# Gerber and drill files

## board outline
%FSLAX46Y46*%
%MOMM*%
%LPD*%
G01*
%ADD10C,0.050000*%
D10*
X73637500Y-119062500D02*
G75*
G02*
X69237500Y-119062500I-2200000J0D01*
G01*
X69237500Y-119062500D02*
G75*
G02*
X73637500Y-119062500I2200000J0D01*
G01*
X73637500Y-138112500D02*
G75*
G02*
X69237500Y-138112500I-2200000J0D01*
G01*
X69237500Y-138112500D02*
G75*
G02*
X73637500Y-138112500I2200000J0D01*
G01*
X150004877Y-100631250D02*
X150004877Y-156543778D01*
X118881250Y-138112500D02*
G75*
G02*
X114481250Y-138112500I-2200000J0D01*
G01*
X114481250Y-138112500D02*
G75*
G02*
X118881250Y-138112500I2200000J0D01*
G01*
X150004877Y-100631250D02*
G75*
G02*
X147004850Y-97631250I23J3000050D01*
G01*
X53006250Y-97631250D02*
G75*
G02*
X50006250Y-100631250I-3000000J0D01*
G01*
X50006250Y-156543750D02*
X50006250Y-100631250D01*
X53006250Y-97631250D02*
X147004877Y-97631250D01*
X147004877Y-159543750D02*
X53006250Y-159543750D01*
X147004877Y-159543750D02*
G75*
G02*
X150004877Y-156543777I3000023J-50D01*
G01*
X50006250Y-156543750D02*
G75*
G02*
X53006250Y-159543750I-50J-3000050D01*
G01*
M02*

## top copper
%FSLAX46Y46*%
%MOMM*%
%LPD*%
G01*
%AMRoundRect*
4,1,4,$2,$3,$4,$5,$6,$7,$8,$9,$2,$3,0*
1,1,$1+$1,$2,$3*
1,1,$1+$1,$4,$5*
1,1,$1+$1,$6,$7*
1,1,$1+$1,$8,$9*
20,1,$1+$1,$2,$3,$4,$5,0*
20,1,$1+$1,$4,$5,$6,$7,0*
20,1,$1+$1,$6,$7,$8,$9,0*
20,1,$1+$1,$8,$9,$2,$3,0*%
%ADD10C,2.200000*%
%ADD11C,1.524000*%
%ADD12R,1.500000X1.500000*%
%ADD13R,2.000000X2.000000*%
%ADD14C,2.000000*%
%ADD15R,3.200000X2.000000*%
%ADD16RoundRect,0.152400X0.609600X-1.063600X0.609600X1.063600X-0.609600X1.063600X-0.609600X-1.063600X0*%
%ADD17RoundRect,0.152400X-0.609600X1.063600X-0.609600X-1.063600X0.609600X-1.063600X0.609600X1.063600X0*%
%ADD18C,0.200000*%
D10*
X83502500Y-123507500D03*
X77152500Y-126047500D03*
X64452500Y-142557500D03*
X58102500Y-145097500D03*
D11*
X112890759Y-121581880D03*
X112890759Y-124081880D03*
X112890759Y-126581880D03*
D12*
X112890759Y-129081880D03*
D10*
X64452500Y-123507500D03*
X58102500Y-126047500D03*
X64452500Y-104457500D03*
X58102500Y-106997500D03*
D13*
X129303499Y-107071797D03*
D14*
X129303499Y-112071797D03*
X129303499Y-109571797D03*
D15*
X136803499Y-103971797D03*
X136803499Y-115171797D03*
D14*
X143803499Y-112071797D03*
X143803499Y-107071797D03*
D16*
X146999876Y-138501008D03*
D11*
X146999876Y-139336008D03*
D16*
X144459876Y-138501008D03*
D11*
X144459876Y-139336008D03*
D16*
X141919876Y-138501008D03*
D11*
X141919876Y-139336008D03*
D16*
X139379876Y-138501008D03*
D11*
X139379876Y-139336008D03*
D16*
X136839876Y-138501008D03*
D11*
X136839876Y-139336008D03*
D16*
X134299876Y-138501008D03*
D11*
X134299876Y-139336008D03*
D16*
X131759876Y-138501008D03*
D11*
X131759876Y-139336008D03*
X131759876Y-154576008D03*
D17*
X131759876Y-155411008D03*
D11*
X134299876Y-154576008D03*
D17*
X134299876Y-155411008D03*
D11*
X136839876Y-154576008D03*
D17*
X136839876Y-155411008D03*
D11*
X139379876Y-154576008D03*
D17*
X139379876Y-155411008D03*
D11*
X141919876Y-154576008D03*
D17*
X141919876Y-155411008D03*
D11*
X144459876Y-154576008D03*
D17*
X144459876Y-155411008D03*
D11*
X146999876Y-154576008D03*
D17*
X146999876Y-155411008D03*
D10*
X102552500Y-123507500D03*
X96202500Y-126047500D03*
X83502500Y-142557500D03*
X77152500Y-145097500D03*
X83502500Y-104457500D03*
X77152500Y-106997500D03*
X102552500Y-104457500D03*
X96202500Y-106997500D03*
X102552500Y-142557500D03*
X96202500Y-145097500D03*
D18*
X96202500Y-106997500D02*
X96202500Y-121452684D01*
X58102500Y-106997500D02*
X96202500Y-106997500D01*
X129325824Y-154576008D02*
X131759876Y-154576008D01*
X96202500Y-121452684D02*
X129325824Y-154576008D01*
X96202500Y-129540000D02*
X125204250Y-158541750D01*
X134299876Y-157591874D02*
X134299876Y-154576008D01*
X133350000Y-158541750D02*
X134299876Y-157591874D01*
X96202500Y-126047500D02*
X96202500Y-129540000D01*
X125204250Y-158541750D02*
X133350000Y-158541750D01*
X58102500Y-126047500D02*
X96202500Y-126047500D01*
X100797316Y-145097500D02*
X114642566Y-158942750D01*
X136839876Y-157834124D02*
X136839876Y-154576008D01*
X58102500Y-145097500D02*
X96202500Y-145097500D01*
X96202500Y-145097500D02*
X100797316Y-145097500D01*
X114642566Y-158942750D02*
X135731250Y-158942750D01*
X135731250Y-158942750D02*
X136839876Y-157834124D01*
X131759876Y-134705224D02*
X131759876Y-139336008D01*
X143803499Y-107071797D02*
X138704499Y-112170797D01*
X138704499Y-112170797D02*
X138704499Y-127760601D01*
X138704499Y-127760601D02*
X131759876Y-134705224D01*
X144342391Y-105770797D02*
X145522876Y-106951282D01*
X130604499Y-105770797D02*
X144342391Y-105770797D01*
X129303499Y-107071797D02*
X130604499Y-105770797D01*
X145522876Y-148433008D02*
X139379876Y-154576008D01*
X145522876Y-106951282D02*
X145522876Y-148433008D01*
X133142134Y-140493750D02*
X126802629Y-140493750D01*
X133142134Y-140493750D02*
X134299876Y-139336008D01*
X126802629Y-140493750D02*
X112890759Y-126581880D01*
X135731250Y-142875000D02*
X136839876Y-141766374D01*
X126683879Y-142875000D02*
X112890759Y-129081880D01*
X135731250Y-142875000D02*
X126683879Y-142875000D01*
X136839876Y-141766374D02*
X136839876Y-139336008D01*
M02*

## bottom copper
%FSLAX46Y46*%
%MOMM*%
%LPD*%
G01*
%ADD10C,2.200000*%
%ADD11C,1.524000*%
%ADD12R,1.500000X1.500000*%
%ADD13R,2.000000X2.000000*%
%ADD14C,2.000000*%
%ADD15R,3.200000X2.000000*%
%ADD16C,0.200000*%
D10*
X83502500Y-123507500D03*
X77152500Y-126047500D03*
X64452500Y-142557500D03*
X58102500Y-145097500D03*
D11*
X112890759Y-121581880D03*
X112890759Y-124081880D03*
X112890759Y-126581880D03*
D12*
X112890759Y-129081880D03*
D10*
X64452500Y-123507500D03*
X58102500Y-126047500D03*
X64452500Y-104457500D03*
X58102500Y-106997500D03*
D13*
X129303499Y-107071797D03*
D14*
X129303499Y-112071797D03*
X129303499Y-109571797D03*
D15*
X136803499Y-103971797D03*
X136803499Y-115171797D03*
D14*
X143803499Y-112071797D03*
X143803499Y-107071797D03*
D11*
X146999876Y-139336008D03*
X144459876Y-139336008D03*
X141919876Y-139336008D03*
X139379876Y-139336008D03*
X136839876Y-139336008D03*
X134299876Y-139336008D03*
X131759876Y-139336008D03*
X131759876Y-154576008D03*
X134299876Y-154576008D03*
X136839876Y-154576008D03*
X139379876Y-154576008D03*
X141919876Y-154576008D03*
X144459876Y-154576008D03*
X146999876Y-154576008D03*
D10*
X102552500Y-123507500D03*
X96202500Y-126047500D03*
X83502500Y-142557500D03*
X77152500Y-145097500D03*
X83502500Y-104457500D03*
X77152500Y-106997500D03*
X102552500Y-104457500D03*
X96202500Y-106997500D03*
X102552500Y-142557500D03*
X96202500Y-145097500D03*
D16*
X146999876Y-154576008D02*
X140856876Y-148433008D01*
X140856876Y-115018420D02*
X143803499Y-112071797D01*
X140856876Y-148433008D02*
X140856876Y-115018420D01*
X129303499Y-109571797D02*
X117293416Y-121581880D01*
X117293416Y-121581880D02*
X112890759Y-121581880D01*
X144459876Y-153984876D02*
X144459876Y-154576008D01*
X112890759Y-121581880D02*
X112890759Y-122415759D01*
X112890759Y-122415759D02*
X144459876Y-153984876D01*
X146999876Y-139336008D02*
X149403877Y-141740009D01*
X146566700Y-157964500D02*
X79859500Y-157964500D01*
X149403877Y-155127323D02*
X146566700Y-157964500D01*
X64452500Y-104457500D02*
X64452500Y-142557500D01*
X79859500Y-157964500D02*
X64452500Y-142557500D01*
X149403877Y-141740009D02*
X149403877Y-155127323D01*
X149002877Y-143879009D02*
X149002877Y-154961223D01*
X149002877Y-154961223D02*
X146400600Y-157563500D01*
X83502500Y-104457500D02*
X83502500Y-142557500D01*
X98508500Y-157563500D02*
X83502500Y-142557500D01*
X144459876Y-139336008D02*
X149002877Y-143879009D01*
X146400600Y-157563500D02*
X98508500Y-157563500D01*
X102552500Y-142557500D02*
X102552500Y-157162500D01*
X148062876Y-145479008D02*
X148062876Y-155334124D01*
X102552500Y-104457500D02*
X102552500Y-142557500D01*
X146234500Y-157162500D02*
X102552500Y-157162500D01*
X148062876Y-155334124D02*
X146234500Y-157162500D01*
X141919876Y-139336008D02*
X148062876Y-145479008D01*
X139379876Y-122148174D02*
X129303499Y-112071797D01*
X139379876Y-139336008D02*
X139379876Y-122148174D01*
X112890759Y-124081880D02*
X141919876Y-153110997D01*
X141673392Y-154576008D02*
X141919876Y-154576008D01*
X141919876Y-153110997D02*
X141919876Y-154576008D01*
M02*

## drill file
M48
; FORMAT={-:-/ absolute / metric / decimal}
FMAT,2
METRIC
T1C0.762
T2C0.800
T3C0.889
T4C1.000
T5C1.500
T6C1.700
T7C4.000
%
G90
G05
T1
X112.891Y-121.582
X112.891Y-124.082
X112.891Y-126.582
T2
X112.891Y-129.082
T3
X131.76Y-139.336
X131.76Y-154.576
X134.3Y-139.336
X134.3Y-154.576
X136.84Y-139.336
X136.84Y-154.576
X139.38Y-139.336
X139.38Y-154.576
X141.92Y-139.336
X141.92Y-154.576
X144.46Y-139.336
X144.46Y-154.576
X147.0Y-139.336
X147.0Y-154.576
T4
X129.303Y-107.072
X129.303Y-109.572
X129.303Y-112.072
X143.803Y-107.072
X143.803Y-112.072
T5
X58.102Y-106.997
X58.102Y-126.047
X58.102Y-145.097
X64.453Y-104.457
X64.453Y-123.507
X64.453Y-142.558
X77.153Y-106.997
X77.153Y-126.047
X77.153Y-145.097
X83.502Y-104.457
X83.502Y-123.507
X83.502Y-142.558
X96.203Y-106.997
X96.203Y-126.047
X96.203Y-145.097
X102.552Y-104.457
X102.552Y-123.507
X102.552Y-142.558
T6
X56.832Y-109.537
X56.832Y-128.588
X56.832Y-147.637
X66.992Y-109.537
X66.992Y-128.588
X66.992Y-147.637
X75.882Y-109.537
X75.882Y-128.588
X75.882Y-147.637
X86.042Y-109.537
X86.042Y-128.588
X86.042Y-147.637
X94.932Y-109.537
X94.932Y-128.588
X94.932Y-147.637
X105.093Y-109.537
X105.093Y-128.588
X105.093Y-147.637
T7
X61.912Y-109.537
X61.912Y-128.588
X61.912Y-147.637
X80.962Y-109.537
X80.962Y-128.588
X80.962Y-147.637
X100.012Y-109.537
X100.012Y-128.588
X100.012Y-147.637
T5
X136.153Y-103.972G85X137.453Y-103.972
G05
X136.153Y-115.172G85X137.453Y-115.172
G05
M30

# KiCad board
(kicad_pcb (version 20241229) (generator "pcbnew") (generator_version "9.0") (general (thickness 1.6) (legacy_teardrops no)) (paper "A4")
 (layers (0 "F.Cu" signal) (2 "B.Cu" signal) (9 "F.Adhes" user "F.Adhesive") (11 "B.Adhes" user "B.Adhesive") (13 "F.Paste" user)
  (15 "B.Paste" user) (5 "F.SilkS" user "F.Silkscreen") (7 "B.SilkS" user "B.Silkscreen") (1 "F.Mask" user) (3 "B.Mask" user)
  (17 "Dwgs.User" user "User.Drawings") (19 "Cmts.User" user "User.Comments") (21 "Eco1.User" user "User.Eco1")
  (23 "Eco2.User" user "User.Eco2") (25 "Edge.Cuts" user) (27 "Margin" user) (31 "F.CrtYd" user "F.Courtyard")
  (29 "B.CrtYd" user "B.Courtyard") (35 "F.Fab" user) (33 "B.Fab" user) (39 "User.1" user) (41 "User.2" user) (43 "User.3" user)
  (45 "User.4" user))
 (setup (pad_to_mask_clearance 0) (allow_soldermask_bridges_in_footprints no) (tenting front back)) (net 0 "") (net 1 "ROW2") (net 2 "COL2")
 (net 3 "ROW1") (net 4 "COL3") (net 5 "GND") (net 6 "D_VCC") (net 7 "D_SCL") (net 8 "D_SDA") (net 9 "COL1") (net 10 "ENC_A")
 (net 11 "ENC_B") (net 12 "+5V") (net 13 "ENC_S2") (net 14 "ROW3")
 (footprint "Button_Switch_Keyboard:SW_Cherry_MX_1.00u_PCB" (layer "F.Cu") (at 83.5025 123.5075)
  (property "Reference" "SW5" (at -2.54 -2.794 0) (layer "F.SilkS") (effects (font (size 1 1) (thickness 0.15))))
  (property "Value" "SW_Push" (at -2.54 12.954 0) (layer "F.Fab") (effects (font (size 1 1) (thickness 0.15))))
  (pad "" np_thru_hole circle (at -7.62 5.08) (size 1.7 1.7) (drill 1.7) (layers "*.Cu" "*.Mask"))
  (pad "" np_thru_hole circle (at -2.54 5.08) (size 4 4) (drill 4) (layers "*.Cu" "*.Mask"))
  (pad "" np_thru_hole circle (at 2.54 5.08) (size 1.7 1.7) (drill 1.7) (layers "*.Cu" "*.Mask"))
  (pad "1" thru_hole circle (at 0 0) (size 2.2 2.2) (drill 1.5) (layers "*.Cu" "*.Mask") (remove_unused_layers no) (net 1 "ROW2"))
  (pad "2" thru_hole circle (at -6.35 2.54) (size 2.2 2.2) (drill 1.5) (layers "*.Cu" "*.Mask") (remove_unused_layers no) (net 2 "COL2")))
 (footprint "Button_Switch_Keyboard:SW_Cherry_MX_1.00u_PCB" (layer "F.Cu") (at 64.4525 142.5575)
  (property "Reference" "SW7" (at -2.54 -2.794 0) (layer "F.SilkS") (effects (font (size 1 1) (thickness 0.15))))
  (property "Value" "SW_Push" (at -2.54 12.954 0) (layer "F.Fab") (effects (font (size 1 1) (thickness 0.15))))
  (pad "" np_thru_hole circle (at -7.62 5.08) (size 1.7 1.7) (drill 1.7) (layers "*.Cu" "*.Mask"))
  (pad "" np_thru_hole circle (at -2.54 5.08) (size 4 4) (drill 4) (layers "*.Cu" "*.Mask"))
  (pad "" np_thru_hole circle (at 2.54 5.08) (size 1.7 1.7) (drill 1.7) (layers "*.Cu" "*.Mask"))
  (pad "1" thru_hole circle (at 0 0) (size 2.2 2.2) (drill 1.5) (layers "*.Cu" "*.Mask") (remove_unused_layers no) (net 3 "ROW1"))
  (pad "2" thru_hole circle (at -6.35 2.54) (size 2.2 2.2) (drill 1.5) (layers "*.Cu" "*.Mask") (remove_unused_layers no) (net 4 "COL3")))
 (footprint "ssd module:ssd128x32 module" (layer "F.Cu") (at 126.12851 139.246137)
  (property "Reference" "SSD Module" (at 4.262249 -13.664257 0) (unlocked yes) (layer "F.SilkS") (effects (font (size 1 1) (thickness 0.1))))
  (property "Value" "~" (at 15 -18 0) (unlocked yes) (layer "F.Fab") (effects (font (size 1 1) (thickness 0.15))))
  (pad "1" thru_hole circle (at -13.237751 -17.664257) (size 1.524 1.524) (drill 0.762) (layers "*.Cu" "*.Mask") (remove_unused_layers no)
   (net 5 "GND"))
  (pad "2" thru_hole circle (at -13.237751 -15.164257) (size 1.524 1.524) (drill 0.762) (layers "*.Cu" "*.Mask") (remove_unused_layers no)
   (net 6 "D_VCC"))
  (pad "3" thru_hole circle (at -13.237751 -12.664257) (size 1.524 1.524) (drill 0.762) (layers "*.Cu" "*.Mask") (remove_unused_layers no)
   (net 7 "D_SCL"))
  (pad "4" thru_hole rect (at -13.237751 -10.164257) (size 1.5 1.5) (drill 0.8) (layers "*.Cu" "*.Mask") (remove_unused_layers no)
   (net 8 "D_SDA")))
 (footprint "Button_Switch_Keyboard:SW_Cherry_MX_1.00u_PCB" (layer "F.Cu") (at 64.4525 123.5075)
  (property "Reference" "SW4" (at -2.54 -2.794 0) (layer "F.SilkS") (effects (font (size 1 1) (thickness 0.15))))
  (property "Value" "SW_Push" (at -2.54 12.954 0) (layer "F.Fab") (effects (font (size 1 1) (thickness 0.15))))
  (pad "" np_thru_hole circle (at -7.62 5.08) (size 1.7 1.7) (drill 1.7) (layers "*.Cu" "*.Mask"))
  (pad "" np_thru_hole circle (at -2.54 5.08) (size 4 4) (drill 4) (layers "*.Cu" "*.Mask"))
  (pad "" np_thru_hole circle (at 2.54 5.08) (size 1.7 1.7) (drill 1.7) (layers "*.Cu" "*.Mask"))
  (pad "1" thru_hole circle (at 0 0) (size 2.2 2.2) (drill 1.5) (layers "*.Cu" "*.Mask") (remove_unused_layers no) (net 3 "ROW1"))
  (pad "2" thru_hole circle (at -6.35 2.54) (size 2.2 2.2) (drill 1.5) (layers "*.Cu" "*.Mask") (remove_unused_layers no) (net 2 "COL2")))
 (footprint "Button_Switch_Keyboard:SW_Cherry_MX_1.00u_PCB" (layer "F.Cu") (at 64.4525 104.4575)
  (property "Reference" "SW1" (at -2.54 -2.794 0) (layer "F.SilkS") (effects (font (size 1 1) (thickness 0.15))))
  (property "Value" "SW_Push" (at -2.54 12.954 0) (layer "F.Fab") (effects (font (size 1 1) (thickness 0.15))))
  (pad "" np_thru_hole circle (at -7.62 5.08) (size 1.7 1.7) (drill 1.7) (layers "*.Cu" "*.Mask"))
  (pad "" np_thru_hole circle (at -2.54 5.08) (size 4 4) (drill 4) (layers "*.Cu" "*.Mask"))
  (pad "" np_thru_hole circle (at 2.54 5.08) (size 1.7 1.7) (drill 1.7) (layers "*.Cu" "*.Mask"))
  (pad "1" thru_hole circle (at 0 0) (size 2.2 2.2) (drill 1.5) (layers "*.Cu" "*.Mask") (remove_unused_layers no) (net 3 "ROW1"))
  (pad "2" thru_hole circle (at -6.35 2.54) (size 2.2 2.2) (drill 1.5) (layers "*.Cu" "*.Mask") (remove_unused_layers no) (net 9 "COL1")))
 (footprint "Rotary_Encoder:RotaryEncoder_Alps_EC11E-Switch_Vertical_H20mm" (layer "F.Cu") (at 129.303499 107.071797)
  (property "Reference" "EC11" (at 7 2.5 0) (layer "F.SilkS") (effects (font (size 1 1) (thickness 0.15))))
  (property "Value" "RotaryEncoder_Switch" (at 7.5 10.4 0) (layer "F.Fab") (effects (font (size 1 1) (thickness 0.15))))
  (pad "A" thru_hole rect (at 0 0) (size 2 2) (drill 1) (layers "*.Cu" "*.Mask") (remove_unused_layers no) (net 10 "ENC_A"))
  (pad "B" thru_hole circle (at 0 5) (size 2 2) (drill 1) (layers "*.Cu" "*.Mask") (remove_unused_layers no) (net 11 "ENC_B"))
  (pad "C" thru_hole circle (at 0 2.5) (size 2 2) (drill 1) (layers "*.Cu" "*.Mask") (remove_unused_layers no) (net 5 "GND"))
  (pad "MP" thru_hole rect (at 7.5 -3.1) (size 3.2 2) (drill oval 2.8 1.5) (layers "*.Cu" "*.Mask") (remove_unused_layers no))
  (pad "MP" thru_hole rect (at 7.5 8.1) (size 3.2 2) (drill oval 2.8 1.5) (layers "*.Cu" "*.Mask") (remove_unused_layers no))
  (pad "S1" thru_hole circle (at 14.5 5) (size 2 2) (drill 1) (layers "*.Cu" "*.Mask") (remove_unused_layers no) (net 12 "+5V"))
  (pad "S2" thru_hole circle (at 14.5 0) (size 2 2) (drill 1) (layers "*.Cu" "*.Mask") (remove_unused_layers no) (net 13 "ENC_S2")))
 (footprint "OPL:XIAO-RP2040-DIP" (layer "F.Cu") (at 139.379876 146.956008 -90)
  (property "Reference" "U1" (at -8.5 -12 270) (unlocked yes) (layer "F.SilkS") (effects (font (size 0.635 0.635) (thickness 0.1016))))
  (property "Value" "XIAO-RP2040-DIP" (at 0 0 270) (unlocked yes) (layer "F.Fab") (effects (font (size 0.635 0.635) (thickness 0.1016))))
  (pad "1" smd roundrect (at -8.455 -7.62 90) (size 2.432 1.524) (layers "F.Cu" "F.Mask") (roundrect_rratio 0.1) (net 3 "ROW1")
   (thermal_bridge_angle 45))
  (pad "1" thru_hole circle (at -7.62 -7.62 90) (size 1.524 1.524) (drill 0.889) (layers "*.Cu" "*.Mask") (remove_unused_layers no)
   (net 3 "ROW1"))
  (pad "2" smd roundrect (at -8.455 -5.08 90) (size 2.432 1.524) (layers "F.Cu" "F.Mask") (roundrect_rratio 0.1) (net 1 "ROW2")
   (thermal_bridge_angle 45))
  (pad "2" thru_hole circle (at -7.62 -5.08 90) (size 1.524 1.524) (drill 0.889) (layers "*.Cu" "*.Mask") (remove_unused_layers no)
   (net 1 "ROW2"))
  (pad "3" smd roundrect (at -8.455 -2.54 90) (size 2.432 1.524) (layers "F.Cu" "F.Mask") (roundrect_rratio 0.1) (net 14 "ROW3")
   (thermal_bridge_angle 45))
  (pad "3" thru_hole circle (at -7.62 -2.54 90) (size 1.524 1.524) (drill 0.889) (layers "*.Cu" "*.Mask") (remove_unused_layers no)
   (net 14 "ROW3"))
  (pad "4" smd roundrect (at -8.455 0 90) (size 2.432 1.524) (layers "F.Cu" "F.Mask") (roundrect_rratio 0.1) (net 11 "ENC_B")
   (thermal_bridge_angle 45))
  (pad "4" thru_hole circle (at -7.62 0 90) (size 1.524 1.524) (drill 0.889) (layers "*.Cu" "*.Mask") (remove_unused_layers no)
   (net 11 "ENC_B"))
  (pad "5" smd roundrect (at -8.455 2.54 90) (size 2.432 1.524) (layers "F.Cu" "F.Mask") (roundrect_rratio 0.1) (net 8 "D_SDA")
   (thermal_bridge_angle 45))
  (pad "5" thru_hole circle (at -7.62 2.54 90) (size 1.524 1.524) (drill 0.889) (layers "*.Cu" "*.Mask") (remove_unused_layers no)
   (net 8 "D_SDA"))
  (pad "6" smd roundrect (at -8.455 5.08 90) (size 2.432 1.524) (layers "F.Cu" "F.Mask") (roundrect_rratio 0.1) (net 7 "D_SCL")
   (thermal_bridge_angle 45))
  (pad "6" thru_hole circle (at -7.62 5.08 90) (size 1.524 1.524) (drill 0.889) (layers "*.Cu" "*.Mask") (remove_unused_layers no)
   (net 7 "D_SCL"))
  (pad "7" smd roundrect (at -8.455 7.62 90) (size 2.432 1.524) (layers "F.Cu" "F.Mask") (roundrect_rratio 0.1) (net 13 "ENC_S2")
   (thermal_bridge_angle 45))
  (pad "7" thru_hole circle (at -7.62 7.62 90) (size 1.524 1.524) (drill 0.889) (layers "*.Cu" "*.Mask") (remove_unused_layers no)
   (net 13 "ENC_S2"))
  (pad "8" thru_hole circle (at 7.62 7.62 270) (size 1.524 1.524) (drill 0.889) (layers "*.Cu" "*.Mask") (remove_unused_layers no)
   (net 9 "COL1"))
  (pad "8" smd roundrect (at 8.455 7.62 270) (size 2.432 1.524) (layers "F.Cu" "F.Mask") (roundrect_rratio 0.1) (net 9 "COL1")
   (thermal_bridge_angle 45))
  (pad "9" thru_hole circle (at 7.62 5.08 270) (size 1.524 1.524) (drill 0.889) (layers "*.Cu" "*.Mask") (remove_unused_layers no)
   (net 2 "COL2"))
  (pad "9" smd roundrect (at 8.455 5.08 270) (size 2.432 1.524) (layers "F.Cu" "F.Mask") (roundrect_rratio 0.1) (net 2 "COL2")
   (thermal_bridge_angle 45))
  (pad "10" thru_hole circle (at 7.62 2.54 270) (size 1.524 1.524) (drill 0.889) (layers "*.Cu" "*.Mask") (remove_unused_layers no)
   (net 4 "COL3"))
  (pad "10" smd roundrect (at 8.455 2.54 270) (size 2.432 1.524) (layers "F.Cu" "F.Mask") (roundrect_rratio 0.1) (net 4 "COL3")
   (thermal_bridge_angle 45))
  (pad "11" thru_hole circle (at 7.62 0 270) (size 1.524 1.524) (drill 0.889) (layers "*.Cu" "*.Mask") (remove_unused_layers no)
   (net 10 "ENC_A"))
  (pad "11" smd roundrect (at 8.455 0 270) (size 2.432 1.524) (layers "F.Cu" "F.Mask") (roundrect_rratio 0.1) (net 10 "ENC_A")
   (thermal_bridge_angle 45))
  (pad "12" thru_hole circle (at 7.62 -2.54 270) (size 1.524 1.524) (drill 0.889) (layers "*.Cu" "*.Mask") (remove_unused_layers no)
   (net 6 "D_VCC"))
  (pad "12" smd roundrect (at 8.455 -2.54 270) (size 2.432 1.524) (layers "F.Cu" "F.Mask") (roundrect_rratio 0.1) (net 6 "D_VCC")
   (thermal_bridge_angle 45))
  (pad "13" thru_hole circle (at 7.62 -5.08 270) (size 1.524 1.524) (drill 0.889) (layers "*.Cu" "*.Mask") (remove_unused_layers no)
   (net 5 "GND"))
  (pad "13" smd roundrect (at 8.455 -5.08 270) (size 2.432 1.524) (layers "F.Cu" "F.Mask") (roundrect_rratio 0.1) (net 5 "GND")
   (thermal_bridge_angle 45))
  (pad "14" thru_hole circle (at 7.62 -7.62 270) (size 1.524 1.524) (drill 0.889) (layers "*.Cu" "*.Mask") (remove_unused_layers no)
   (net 12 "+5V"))
  (pad "14" smd roundrect (at 8.455 -7.62 270) (size 2.432 1.524) (layers "F.Cu" "F.Mask") (roundrect_rratio 0.1) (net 12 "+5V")
   (thermal_bridge_angle 45)))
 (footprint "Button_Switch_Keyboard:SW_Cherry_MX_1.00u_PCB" (layer "F.Cu") (at 102.5525 123.5075)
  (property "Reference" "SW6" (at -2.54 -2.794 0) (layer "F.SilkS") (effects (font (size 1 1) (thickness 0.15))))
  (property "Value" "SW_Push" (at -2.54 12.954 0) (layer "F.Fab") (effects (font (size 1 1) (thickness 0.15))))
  (pad "" np_thru_hole circle (at -7.62 5.08) (size 1.7 1.7) (drill 1.7) (layers "*.Cu" "*.Mask"))
  (pad "" np_thru_hole circle (at -2.54 5.08) (size 4 4) (drill 4) (layers "*.Cu" "*.Mask"))
  (pad "" np_thru_hole circle (at 2.54 5.08) (size 1.7 1.7) (drill 1.7) (layers "*.Cu" "*.Mask"))
  (pad "1" thru_hole circle (at 0 0) (size 2.2 2.2) (drill 1.5) (layers "*.Cu" "*.Mask") (remove_unused_layers no) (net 14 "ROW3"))
  (pad "2" thru_hole circle (at -6.35 2.54) (size 2.2 2.2) (drill 1.5) (layers "*.Cu" "*.Mask") (remove_unused_layers no) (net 2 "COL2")))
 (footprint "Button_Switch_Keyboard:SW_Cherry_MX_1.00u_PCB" (layer "F.Cu") (at 83.5025 142.5575)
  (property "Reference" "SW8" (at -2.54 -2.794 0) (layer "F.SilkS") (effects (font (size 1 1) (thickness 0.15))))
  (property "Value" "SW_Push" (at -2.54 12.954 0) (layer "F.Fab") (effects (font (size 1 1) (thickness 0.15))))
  (pad "" np_thru_hole circle (at -7.62 5.08) (size 1.7 1.7) (drill 1.7) (layers "*.Cu" "*.Mask"))
  (pad "" np_thru_hole circle (at -2.54 5.08) (size 4 4) (drill 4) (layers "*.Cu" "*.Mask"))
  (pad "" np_thru_hole circle (at 2.54 5.08) (size 1.7 1.7) (drill 1.7) (layers "*.Cu" "*.Mask"))
  (pad "1" thru_hole circle (at 0 0) (size 2.2 2.2) (drill 1.5) (layers "*.Cu" "*.Mask") (remove_unused_layers no) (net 1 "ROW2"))
  (pad "2" thru_hole circle (at -6.35 2.54) (size 2.2 2.2) (drill 1.5) (layers "*.Cu" "*.Mask") (remove_unused_layers no) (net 4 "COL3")))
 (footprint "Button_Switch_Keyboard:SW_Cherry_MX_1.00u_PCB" (layer "F.Cu") (at 83.5025 104.4575)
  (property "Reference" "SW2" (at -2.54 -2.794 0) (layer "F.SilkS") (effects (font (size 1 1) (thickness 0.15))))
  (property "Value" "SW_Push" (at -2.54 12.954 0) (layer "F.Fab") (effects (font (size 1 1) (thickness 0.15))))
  (pad "" np_thru_hole circle (at -7.62 5.08) (size 1.7 1.7) (drill 1.7) (layers "*.Cu" "*.Mask"))
  (pad "" np_thru_hole circle (at -2.54 5.08) (size 4 4) (drill 4) (layers "*.Cu" "*.Mask"))
  (pad "" np_thru_hole circle (at 2.54 5.08) (size 1.7 1.7) (drill 1.7) (layers "*.Cu" "*.Mask"))
  (pad "1" thru_hole circle (at 0 0) (size 2.2 2.2) (drill 1.5) (layers "*.Cu" "*.Mask") (remove_unused_layers no) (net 1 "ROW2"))
  (pad "2" thru_hole circle (at -6.35 2.54) (size 2.2 2.2) (drill 1.5) (layers "*.Cu" "*.Mask") (remove_unused_layers no) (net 9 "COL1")))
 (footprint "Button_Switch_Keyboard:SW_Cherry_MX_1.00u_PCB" (layer "F.Cu") (at 102.5525 104.4575)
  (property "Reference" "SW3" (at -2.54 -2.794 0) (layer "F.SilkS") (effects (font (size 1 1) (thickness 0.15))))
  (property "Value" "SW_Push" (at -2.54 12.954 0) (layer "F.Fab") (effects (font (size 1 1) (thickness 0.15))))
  (pad "" np_thru_hole circle (at -7.62 5.08) (size 1.7 1.7) (drill 1.7) (layers "*.Cu" "*.Mask"))
  (pad "" np_thru_hole circle (at -2.54 5.08) (size 4 4) (drill 4) (layers "*.Cu" "*.Mask"))
  (pad "" np_thru_hole circle (at 2.54 5.08) (size 1.7 1.7) (drill 1.7) (layers "*.Cu" "*.Mask"))
  (pad "1" thru_hole circle (at 0 0) (size 2.2 2.2) (drill 1.5) (layers "*.Cu" "*.Mask") (remove_unused_layers no) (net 14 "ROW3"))
  (pad "2" thru_hole circle (at -6.35 2.54) (size 2.2 2.2) (drill 1.5) (layers "*.Cu" "*.Mask") (remove_unused_layers no) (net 9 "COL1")))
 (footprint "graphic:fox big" (layer "F.Cu") (at 119.0625 109.5375)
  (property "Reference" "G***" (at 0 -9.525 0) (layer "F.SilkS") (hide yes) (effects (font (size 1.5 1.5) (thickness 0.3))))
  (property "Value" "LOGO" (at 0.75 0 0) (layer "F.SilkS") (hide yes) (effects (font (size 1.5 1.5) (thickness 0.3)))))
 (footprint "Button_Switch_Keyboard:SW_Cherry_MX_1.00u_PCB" (layer "F.Cu") (at 102.5525 142.5575)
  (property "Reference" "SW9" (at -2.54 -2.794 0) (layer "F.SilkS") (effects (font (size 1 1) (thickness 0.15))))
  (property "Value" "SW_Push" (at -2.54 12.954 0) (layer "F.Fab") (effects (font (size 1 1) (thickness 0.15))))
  (pad "" np_thru_hole circle (at -7.62 5.08) (size 1.7 1.7) (drill 1.7) (layers "*.Cu" "*.Mask"))
  (pad "" np_thru_hole circle (at -2.54 5.08) (size 4 4) (drill 4) (layers "*.Cu" "*.Mask"))
  (pad "" np_thru_hole circle (at 2.54 5.08) (size 1.7 1.7) (drill 1.7) (layers "*.Cu" "*.Mask"))
  (pad "1" thru_hole circle (at 0 0) (size 2.2 2.2) (drill 1.5) (layers "*.Cu" "*.Mask") (remove_unused_layers no) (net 14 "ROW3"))
  (pad "2" thru_hole circle (at -6.35 2.54) (size 2.2 2.2) (drill 1.5) (layers "*.Cu" "*.Mask") (remove_unused_layers no) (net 4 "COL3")))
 (gr_circle (center 71.4375 119.0625) (end 73.6375 119.0625) (stroke (width 0.05) (type solid)) (fill no) (layer "Edge.Cuts"))
 (gr_circle (center 71.4375 138.1125) (end 73.6375 138.1125) (stroke (width 0.05) (type solid)) (fill no) (layer "Edge.Cuts"))
 (gr_line (start 150.004877 100.63125) (end 150.004877 156.543778) (stroke (width 0.05) (type default)) (layer "Edge.Cuts"))
 (gr_circle (center 116.68125 138.1125) (end 118.88125 138.1125) (stroke (width 0.05) (type solid)) (fill no) (layer "Edge.Cuts"))
 (gr_arc (start 150.004877 100.63125) (mid 147.883557 99.75257) (end 147.004877 97.63125) (stroke (width 0.05) (type default))
  (layer "Edge.Cuts"))
 (gr_arc (start 53.00625 97.63125) (mid 52.12757 99.75257) (end 50.00625 100.63125) (stroke (width 0.05) (type default)) (layer "Edge.Cuts"))
 (gr_line (start 50.00625 156.54375) (end 50.00625 100.63125) (stroke (width 0.05) (type default)) (layer "Edge.Cuts"))
 (gr_line (start 53.00625 97.63125) (end 147.004877 97.63125) (stroke (width 0.05) (type default)) (layer "Edge.Cuts"))
 (gr_line (start 147.004877 159.54375) (end 53.00625 159.54375) (stroke (width 0.05) (type default)) (layer "Edge.Cuts"))
 (gr_arc (start 147.004877 159.54375) (mid 147.883557 157.42243) (end 150.004877 156.54375) (stroke (width 0.05) (type default))
  (layer "Edge.Cuts"))
 (gr_arc (start 50.00625 156.54375) (mid 52.12757 157.42243) (end 53.00625 159.54375) (stroke (width 0.05) (type default))
  (layer "Edge.Cuts"))
 (segment (start 146.999876 154.576008) (end 140.856876 148.433008) (width 0.2) (layer "B.Cu") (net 12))
 (segment (start 140.856876 115.01842) (end 143.803499 112.071797) (width 0.2) (layer "B.Cu") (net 12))
 (segment (start 140.856876 148.433008) (end 140.856876 115.01842) (width 0.2) (layer "B.Cu") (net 12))
 (segment (start 129.303499 109.571797) (end 117.293416 121.58188) (width 0.2) (layer "B.Cu") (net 5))
 (segment (start 117.293416 121.58188) (end 112.890759 121.58188) (width 0.2) (layer "B.Cu") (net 5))
 (segment (start 144.459876 153.984876) (end 144.459876 154.576008) (width 0.2) (layer "B.Cu") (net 5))
 (segment (start 112.890759 121.58188) (end 112.890759 122.415759) (width 0.2) (layer "B.Cu") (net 5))
 (segment (start 112.890759 122.415759) (end 144.459876 153.984876) (width 0.2) (layer "B.Cu") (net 5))
 (segment (start 146.999876 139.336008) (end 149.403877 141.740009) (width 0.2) (layer "B.Cu") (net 3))
 (segment (start 146.5667 157.9645) (end 79.8595 157.9645) (width 0.2) (layer "B.Cu") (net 3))
 (segment (start 149.403877 155.127323) (end 146.5667 157.9645) (width 0.2) (layer "B.Cu") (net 3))
 (segment (start 64.4525 104.4575) (end 64.4525 142.5575) (width 0.2) (layer "B.Cu") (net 3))
 (segment (start 79.8595 157.9645) (end 64.4525 142.5575) (width 0.2) (layer "B.Cu") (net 3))
 (segment (start 149.403877 141.740009) (end 149.403877 155.127323) (width 0.2) (layer "B.Cu") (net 3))
 (segment (start 96.2025 106.9975) (end 96.2025 121.452684) (width 0.2) (layer "F.Cu") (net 9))
 (segment (start 58.1025 106.9975) (end 96.2025 106.9975) (width 0.2) (layer "F.Cu") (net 9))
 (segment (start 129.325824 154.576008) (end 131.759876 154.576008) (width 0.2) (layer "F.Cu") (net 9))
 (segment (start 96.2025 121.452684) (end 129.325824 154.576008) (width 0.2) (layer "F.Cu") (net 9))
 (segment (start 149.002877 143.879009) (end 149.002877 154.961223) (width 0.2) (layer "B.Cu") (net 1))
 (segment (start 149.002877 154.961223) (end 146.4006 157.5635) (width 0.2) (layer "B.Cu") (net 1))
 (segment (start 83.5025 104.4575) (end 83.5025 142.5575) (width 0.2) (layer "B.Cu") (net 1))
 (segment (start 98.5085 157.5635) (end 83.5025 142.5575) (width 0.2) (layer "B.Cu") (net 1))
 (segment (start 144.459876 139.336008) (end 149.002877 143.879009) (width 0.2) (layer "B.Cu") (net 1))
 (segment (start 146.4006 157.5635) (end 98.5085 157.5635) (width 0.2) (layer "B.Cu") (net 1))
 (segment (start 102.5525 142.5575) (end 102.5525 157.1625) (width 0.2) (layer "B.Cu") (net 14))
 (segment (start 148.062876 145.479008) (end 148.062876 155.334124) (width 0.2) (layer "B.Cu") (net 14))
 (segment (start 102.5525 104.4575) (end 102.5525 142.5575) (width 0.2) (layer "B.Cu") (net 14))
 (segment (start 146.2345 157.1625) (end 102.5525 157.1625) (width 0.2) (layer "B.Cu") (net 14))
 (segment (start 148.062876 155.334124) (end 146.2345 157.1625) (width 0.2) (layer "B.Cu") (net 14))
 (segment (start 141.919876 139.336008) (end 148.062876 145.479008) (width 0.2) (layer "B.Cu") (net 14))
 (segment (start 96.2025 129.54) (end 125.20425 158.54175) (width 0.2) (layer "F.Cu") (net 2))
 (segment (start 134.299876 157.591874) (end 134.299876 154.576008) (width 0.2) (layer "F.Cu") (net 2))
 (segment (start 133.35 158.54175) (end 134.299876 157.591874) (width 0.2) (layer "F.Cu") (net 2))
 (segment (start 96.2025 126.0475) (end 96.2025 129.54) (width 0.2) (layer "F.Cu") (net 2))
 (segment (start 125.20425 158.54175) (end 133.35 158.54175) (width 0.2) (layer "F.Cu") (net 2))
 (segment (start 58.1025 126.0475) (end 96.2025 126.0475) (width 0.2) (layer "F.Cu") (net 2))
 (segment (start 100.797316 145.0975) (end 114.642566 158.94275) (width 0.2) (layer "F.Cu") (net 4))
 (segment (start 136.839876 157.834124) (end 136.839876 154.576008) (width 0.2) (layer "F.Cu") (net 4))
 (segment (start 58.1025 145.0975) (end 96.2025 145.0975) (width 0.2) (layer "F.Cu") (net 4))
 (segment (start 96.2025 145.0975) (end 100.797316 145.0975) (width 0.2) (layer "F.Cu") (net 4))
 (segment (start 114.642566 158.94275) (end 135.73125 158.94275) (width 0.2) (layer "F.Cu") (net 4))
 (segment (start 135.73125 158.94275) (end 136.839876 157.834124) (width 0.2) (layer "F.Cu") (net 4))
 (segment (start 131.759876 134.705224) (end 131.759876 139.336008) (width 0.2) (layer "F.Cu") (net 13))
 (segment (start 143.803499 107.071797) (end 138.704499 112.170797) (width 0.2) (layer "F.Cu") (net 13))
 (segment (start 138.704499 112.170797) (end 138.704499 127.760601) (width 0.2) (layer "F.Cu") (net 13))
 (segment (start 138.704499 127.760601) (end 131.759876 134.705224) (width 0.2) (layer "F.Cu") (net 13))
 (segment (start 139.379876 122.148174) (end 129.303499 112.071797) (width 0.2) (layer "B.Cu") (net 11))
 (segment (start 139.379876 139.336008) (end 139.379876 122.148174) (width 0.2) (layer "B.Cu") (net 11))
 (segment (start 144.342391 105.770797) (end 145.522876 106.951282) (width 0.2) (layer "F.Cu") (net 10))
 (segment (start 130.604499 105.770797) (end 144.342391 105.770797) (width 0.2) (layer "F.Cu") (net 10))
 (segment (start 129.303499 107.071797) (end 130.604499 105.770797) (width 0.2) (layer "F.Cu") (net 10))
 (segment (start 145.522876 148.433008) (end 139.379876 154.576008) (width 0.2) (layer "F.Cu") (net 10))
 (segment (start 145.522876 106.951282) (end 145.522876 148.433008) (width 0.2) (layer "F.Cu") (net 10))
 (segment (start 133.142134 140.49375) (end 126.802629 140.49375) (width 0.2) (layer "F.Cu") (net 7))
 (segment (start 133.142134 140.49375) (end 134.299876 139.336008) (width 0.2) (layer "F.Cu") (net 7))
 (segment (start 126.802629 140.49375) (end 112.890759 126.58188) (width 0.2) (layer "F.Cu") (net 7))
 (segment (start 135.73125 142.875) (end 136.839876 141.766374) (width 0.2) (layer "F.Cu") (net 8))
 (segment (start 126.683879 142.875) (end 112.890759 129.08188) (width 0.2) (layer "F.Cu") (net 8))
 (segment (start 135.73125 142.875) (end 126.683879 142.875) (width 0.2) (layer "F.Cu") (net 8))
 (segment (start 136.839876 141.766374) (end 136.839876 139.336008) (width 0.2) (layer "F.Cu") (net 8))
 (segment (start 112.890759 124.08188) (end 141.919876 153.110997) (width 0.2) (layer "B.Cu") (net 6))
 (segment (start 141.673392 154.576008) (end 141.919876 154.576008) (width 0.2) (layer "B.Cu") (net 6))
 (segment (start 141.919876 153.110997) (end 141.919876 154.576008) (width 0.2) (layer "B.Cu") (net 6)))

